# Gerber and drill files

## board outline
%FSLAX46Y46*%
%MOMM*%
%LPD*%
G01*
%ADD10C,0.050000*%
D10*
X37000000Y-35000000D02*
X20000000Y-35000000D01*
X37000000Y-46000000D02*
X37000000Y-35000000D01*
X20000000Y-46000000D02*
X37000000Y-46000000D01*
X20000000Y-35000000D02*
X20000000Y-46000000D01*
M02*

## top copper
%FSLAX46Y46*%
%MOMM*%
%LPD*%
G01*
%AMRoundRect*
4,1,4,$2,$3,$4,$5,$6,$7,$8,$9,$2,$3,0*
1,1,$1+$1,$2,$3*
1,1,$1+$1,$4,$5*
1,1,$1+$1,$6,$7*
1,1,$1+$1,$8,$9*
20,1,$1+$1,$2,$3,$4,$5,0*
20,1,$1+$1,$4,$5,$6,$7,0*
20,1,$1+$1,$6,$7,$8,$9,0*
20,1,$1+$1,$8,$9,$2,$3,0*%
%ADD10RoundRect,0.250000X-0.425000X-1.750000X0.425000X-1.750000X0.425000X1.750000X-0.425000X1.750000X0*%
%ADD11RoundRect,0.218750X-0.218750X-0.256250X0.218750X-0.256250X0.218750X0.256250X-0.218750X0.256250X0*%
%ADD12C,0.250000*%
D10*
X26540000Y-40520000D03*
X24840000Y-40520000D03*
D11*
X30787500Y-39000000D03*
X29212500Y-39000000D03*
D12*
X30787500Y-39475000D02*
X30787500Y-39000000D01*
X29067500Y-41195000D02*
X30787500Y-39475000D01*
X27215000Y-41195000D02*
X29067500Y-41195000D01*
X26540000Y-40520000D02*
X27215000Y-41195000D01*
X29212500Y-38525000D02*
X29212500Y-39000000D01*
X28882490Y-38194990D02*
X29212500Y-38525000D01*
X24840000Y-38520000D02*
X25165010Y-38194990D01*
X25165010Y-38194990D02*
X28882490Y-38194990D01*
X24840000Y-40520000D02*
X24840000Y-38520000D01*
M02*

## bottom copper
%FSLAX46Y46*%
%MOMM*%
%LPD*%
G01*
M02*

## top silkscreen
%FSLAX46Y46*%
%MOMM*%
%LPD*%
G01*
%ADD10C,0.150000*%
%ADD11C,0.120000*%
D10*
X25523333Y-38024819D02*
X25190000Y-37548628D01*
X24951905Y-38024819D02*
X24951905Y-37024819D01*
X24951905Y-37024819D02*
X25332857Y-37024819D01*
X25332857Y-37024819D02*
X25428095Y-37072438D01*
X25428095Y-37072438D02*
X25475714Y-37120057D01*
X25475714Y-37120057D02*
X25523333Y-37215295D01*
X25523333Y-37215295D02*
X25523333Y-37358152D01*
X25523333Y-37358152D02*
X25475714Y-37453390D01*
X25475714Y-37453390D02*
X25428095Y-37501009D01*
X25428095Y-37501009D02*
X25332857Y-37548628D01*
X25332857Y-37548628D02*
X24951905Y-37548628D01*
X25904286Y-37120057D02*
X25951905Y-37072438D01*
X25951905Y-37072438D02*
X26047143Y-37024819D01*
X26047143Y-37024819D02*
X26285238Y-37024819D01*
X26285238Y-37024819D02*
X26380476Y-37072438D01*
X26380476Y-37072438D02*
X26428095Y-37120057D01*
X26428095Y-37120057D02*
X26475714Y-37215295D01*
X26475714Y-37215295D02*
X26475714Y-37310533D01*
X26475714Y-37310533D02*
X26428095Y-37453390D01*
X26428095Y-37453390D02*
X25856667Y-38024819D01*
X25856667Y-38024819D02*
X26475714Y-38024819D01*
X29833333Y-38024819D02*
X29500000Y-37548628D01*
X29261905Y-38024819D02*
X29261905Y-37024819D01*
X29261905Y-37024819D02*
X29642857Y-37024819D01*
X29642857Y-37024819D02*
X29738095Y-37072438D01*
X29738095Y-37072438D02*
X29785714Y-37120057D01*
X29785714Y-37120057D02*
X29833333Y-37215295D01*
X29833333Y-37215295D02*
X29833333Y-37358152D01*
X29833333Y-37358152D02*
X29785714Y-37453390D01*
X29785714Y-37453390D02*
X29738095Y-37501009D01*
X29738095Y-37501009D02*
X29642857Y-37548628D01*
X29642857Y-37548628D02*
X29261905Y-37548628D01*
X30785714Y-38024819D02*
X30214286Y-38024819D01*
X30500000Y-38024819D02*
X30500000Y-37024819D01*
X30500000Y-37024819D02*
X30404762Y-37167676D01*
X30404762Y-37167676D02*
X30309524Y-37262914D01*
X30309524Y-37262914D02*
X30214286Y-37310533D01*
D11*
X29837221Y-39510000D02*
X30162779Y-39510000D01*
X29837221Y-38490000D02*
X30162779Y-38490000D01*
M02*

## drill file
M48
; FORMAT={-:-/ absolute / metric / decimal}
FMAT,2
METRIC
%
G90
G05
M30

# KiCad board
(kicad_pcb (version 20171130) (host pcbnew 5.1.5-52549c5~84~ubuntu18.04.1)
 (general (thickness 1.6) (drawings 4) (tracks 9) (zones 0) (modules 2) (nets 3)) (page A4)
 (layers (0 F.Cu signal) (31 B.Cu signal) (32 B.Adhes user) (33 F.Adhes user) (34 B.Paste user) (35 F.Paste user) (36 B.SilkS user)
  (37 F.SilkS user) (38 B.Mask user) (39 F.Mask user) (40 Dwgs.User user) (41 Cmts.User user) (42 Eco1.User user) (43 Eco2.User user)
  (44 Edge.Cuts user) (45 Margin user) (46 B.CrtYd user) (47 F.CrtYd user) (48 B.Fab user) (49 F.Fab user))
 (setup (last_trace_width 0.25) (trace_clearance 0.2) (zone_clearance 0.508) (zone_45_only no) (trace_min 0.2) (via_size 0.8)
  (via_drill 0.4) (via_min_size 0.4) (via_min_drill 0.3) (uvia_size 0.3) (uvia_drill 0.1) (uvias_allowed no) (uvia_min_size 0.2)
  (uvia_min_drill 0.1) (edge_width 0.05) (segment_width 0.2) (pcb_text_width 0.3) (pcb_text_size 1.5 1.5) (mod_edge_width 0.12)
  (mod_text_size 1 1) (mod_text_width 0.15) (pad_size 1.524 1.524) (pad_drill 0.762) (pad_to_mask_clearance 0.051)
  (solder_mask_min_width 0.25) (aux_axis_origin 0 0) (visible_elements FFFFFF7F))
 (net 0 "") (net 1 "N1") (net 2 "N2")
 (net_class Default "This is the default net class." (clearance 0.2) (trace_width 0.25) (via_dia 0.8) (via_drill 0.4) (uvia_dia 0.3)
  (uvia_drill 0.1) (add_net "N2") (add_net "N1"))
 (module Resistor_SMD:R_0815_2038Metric (layer F.Cu) (at 25.69 40.52)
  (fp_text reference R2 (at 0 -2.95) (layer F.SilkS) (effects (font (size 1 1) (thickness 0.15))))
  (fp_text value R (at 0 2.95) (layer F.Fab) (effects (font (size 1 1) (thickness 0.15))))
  (pad 2 smd roundrect (at 0.85 0) (size 1.35 4) (layers F.Cu F.Paste F.Mask) (roundrect_rratio 0.185185) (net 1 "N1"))
  (pad 1 smd roundrect (at -0.85 0) (size 1.35 4) (layers F.Cu F.Paste F.Mask) (roundrect_rratio 0.185185) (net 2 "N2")))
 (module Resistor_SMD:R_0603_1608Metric (layer F.Cu) (at 30 39)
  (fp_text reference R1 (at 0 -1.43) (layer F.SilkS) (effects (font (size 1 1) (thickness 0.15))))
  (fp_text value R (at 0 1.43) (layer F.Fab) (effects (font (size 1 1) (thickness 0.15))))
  (fp_line (start -0.162779 0.51) (end 0.162779 0.51) (layer F.SilkS) (width 0.12))
  (fp_line (start -0.162779 -0.51) (end 0.162779 -0.51) (layer F.SilkS) (width 0.12))
  (pad 2 smd roundrect (at 0.7875 0) (size 0.875 0.95) (layers F.Cu F.Paste F.Mask) (roundrect_rratio 0.25) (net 1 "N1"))
  (pad 1 smd roundrect (at -0.7875 0) (size 0.875 0.95) (layers F.Cu F.Paste F.Mask) (roundrect_rratio 0.25) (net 2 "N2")))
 (gr_line (start 37 35) (end 20 35) (layer Edge.Cuts) (width 0.05))
 (gr_line (start 37 46) (end 37 35) (layer Edge.Cuts) (width 0.05))
 (gr_line (start 20 46) (end 37 46) (layer Edge.Cuts) (width 0.05))
 (gr_line (start 20 35) (end 20 46) (layer Edge.Cuts) (width 0.05))
 (segment (start 30.7875 39.475) (end 30.7875 39) (width 0.25) (layer F.Cu) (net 1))
 (segment (start 29.0675 41.195) (end 30.7875 39.475) (width 0.25) (layer F.Cu) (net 1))
 (segment (start 27.215 41.195) (end 29.0675 41.195) (width 0.25) (layer F.Cu) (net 1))
 (segment (start 26.54 40.52) (end 27.215 41.195) (width 0.25) (layer F.Cu) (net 1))
 (segment (start 29.2125 38.525) (end 29.2125 39) (width 0.25) (layer F.Cu) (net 2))
 (segment (start 28.88249 38.19499) (end 29.2125 38.525) (width 0.25) (layer F.Cu) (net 2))
 (segment (start 24.84 38.52) (end 25.16501 38.19499) (width 0.25) (layer F.Cu) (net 2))
 (segment (start 25.16501 38.19499) (end 28.88249 38.19499) (width 0.25) (layer F.Cu) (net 2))
 (segment (start 24.84 40.52) (end 24.84 38.52) (width 0.25) (layer F.Cu) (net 2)))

